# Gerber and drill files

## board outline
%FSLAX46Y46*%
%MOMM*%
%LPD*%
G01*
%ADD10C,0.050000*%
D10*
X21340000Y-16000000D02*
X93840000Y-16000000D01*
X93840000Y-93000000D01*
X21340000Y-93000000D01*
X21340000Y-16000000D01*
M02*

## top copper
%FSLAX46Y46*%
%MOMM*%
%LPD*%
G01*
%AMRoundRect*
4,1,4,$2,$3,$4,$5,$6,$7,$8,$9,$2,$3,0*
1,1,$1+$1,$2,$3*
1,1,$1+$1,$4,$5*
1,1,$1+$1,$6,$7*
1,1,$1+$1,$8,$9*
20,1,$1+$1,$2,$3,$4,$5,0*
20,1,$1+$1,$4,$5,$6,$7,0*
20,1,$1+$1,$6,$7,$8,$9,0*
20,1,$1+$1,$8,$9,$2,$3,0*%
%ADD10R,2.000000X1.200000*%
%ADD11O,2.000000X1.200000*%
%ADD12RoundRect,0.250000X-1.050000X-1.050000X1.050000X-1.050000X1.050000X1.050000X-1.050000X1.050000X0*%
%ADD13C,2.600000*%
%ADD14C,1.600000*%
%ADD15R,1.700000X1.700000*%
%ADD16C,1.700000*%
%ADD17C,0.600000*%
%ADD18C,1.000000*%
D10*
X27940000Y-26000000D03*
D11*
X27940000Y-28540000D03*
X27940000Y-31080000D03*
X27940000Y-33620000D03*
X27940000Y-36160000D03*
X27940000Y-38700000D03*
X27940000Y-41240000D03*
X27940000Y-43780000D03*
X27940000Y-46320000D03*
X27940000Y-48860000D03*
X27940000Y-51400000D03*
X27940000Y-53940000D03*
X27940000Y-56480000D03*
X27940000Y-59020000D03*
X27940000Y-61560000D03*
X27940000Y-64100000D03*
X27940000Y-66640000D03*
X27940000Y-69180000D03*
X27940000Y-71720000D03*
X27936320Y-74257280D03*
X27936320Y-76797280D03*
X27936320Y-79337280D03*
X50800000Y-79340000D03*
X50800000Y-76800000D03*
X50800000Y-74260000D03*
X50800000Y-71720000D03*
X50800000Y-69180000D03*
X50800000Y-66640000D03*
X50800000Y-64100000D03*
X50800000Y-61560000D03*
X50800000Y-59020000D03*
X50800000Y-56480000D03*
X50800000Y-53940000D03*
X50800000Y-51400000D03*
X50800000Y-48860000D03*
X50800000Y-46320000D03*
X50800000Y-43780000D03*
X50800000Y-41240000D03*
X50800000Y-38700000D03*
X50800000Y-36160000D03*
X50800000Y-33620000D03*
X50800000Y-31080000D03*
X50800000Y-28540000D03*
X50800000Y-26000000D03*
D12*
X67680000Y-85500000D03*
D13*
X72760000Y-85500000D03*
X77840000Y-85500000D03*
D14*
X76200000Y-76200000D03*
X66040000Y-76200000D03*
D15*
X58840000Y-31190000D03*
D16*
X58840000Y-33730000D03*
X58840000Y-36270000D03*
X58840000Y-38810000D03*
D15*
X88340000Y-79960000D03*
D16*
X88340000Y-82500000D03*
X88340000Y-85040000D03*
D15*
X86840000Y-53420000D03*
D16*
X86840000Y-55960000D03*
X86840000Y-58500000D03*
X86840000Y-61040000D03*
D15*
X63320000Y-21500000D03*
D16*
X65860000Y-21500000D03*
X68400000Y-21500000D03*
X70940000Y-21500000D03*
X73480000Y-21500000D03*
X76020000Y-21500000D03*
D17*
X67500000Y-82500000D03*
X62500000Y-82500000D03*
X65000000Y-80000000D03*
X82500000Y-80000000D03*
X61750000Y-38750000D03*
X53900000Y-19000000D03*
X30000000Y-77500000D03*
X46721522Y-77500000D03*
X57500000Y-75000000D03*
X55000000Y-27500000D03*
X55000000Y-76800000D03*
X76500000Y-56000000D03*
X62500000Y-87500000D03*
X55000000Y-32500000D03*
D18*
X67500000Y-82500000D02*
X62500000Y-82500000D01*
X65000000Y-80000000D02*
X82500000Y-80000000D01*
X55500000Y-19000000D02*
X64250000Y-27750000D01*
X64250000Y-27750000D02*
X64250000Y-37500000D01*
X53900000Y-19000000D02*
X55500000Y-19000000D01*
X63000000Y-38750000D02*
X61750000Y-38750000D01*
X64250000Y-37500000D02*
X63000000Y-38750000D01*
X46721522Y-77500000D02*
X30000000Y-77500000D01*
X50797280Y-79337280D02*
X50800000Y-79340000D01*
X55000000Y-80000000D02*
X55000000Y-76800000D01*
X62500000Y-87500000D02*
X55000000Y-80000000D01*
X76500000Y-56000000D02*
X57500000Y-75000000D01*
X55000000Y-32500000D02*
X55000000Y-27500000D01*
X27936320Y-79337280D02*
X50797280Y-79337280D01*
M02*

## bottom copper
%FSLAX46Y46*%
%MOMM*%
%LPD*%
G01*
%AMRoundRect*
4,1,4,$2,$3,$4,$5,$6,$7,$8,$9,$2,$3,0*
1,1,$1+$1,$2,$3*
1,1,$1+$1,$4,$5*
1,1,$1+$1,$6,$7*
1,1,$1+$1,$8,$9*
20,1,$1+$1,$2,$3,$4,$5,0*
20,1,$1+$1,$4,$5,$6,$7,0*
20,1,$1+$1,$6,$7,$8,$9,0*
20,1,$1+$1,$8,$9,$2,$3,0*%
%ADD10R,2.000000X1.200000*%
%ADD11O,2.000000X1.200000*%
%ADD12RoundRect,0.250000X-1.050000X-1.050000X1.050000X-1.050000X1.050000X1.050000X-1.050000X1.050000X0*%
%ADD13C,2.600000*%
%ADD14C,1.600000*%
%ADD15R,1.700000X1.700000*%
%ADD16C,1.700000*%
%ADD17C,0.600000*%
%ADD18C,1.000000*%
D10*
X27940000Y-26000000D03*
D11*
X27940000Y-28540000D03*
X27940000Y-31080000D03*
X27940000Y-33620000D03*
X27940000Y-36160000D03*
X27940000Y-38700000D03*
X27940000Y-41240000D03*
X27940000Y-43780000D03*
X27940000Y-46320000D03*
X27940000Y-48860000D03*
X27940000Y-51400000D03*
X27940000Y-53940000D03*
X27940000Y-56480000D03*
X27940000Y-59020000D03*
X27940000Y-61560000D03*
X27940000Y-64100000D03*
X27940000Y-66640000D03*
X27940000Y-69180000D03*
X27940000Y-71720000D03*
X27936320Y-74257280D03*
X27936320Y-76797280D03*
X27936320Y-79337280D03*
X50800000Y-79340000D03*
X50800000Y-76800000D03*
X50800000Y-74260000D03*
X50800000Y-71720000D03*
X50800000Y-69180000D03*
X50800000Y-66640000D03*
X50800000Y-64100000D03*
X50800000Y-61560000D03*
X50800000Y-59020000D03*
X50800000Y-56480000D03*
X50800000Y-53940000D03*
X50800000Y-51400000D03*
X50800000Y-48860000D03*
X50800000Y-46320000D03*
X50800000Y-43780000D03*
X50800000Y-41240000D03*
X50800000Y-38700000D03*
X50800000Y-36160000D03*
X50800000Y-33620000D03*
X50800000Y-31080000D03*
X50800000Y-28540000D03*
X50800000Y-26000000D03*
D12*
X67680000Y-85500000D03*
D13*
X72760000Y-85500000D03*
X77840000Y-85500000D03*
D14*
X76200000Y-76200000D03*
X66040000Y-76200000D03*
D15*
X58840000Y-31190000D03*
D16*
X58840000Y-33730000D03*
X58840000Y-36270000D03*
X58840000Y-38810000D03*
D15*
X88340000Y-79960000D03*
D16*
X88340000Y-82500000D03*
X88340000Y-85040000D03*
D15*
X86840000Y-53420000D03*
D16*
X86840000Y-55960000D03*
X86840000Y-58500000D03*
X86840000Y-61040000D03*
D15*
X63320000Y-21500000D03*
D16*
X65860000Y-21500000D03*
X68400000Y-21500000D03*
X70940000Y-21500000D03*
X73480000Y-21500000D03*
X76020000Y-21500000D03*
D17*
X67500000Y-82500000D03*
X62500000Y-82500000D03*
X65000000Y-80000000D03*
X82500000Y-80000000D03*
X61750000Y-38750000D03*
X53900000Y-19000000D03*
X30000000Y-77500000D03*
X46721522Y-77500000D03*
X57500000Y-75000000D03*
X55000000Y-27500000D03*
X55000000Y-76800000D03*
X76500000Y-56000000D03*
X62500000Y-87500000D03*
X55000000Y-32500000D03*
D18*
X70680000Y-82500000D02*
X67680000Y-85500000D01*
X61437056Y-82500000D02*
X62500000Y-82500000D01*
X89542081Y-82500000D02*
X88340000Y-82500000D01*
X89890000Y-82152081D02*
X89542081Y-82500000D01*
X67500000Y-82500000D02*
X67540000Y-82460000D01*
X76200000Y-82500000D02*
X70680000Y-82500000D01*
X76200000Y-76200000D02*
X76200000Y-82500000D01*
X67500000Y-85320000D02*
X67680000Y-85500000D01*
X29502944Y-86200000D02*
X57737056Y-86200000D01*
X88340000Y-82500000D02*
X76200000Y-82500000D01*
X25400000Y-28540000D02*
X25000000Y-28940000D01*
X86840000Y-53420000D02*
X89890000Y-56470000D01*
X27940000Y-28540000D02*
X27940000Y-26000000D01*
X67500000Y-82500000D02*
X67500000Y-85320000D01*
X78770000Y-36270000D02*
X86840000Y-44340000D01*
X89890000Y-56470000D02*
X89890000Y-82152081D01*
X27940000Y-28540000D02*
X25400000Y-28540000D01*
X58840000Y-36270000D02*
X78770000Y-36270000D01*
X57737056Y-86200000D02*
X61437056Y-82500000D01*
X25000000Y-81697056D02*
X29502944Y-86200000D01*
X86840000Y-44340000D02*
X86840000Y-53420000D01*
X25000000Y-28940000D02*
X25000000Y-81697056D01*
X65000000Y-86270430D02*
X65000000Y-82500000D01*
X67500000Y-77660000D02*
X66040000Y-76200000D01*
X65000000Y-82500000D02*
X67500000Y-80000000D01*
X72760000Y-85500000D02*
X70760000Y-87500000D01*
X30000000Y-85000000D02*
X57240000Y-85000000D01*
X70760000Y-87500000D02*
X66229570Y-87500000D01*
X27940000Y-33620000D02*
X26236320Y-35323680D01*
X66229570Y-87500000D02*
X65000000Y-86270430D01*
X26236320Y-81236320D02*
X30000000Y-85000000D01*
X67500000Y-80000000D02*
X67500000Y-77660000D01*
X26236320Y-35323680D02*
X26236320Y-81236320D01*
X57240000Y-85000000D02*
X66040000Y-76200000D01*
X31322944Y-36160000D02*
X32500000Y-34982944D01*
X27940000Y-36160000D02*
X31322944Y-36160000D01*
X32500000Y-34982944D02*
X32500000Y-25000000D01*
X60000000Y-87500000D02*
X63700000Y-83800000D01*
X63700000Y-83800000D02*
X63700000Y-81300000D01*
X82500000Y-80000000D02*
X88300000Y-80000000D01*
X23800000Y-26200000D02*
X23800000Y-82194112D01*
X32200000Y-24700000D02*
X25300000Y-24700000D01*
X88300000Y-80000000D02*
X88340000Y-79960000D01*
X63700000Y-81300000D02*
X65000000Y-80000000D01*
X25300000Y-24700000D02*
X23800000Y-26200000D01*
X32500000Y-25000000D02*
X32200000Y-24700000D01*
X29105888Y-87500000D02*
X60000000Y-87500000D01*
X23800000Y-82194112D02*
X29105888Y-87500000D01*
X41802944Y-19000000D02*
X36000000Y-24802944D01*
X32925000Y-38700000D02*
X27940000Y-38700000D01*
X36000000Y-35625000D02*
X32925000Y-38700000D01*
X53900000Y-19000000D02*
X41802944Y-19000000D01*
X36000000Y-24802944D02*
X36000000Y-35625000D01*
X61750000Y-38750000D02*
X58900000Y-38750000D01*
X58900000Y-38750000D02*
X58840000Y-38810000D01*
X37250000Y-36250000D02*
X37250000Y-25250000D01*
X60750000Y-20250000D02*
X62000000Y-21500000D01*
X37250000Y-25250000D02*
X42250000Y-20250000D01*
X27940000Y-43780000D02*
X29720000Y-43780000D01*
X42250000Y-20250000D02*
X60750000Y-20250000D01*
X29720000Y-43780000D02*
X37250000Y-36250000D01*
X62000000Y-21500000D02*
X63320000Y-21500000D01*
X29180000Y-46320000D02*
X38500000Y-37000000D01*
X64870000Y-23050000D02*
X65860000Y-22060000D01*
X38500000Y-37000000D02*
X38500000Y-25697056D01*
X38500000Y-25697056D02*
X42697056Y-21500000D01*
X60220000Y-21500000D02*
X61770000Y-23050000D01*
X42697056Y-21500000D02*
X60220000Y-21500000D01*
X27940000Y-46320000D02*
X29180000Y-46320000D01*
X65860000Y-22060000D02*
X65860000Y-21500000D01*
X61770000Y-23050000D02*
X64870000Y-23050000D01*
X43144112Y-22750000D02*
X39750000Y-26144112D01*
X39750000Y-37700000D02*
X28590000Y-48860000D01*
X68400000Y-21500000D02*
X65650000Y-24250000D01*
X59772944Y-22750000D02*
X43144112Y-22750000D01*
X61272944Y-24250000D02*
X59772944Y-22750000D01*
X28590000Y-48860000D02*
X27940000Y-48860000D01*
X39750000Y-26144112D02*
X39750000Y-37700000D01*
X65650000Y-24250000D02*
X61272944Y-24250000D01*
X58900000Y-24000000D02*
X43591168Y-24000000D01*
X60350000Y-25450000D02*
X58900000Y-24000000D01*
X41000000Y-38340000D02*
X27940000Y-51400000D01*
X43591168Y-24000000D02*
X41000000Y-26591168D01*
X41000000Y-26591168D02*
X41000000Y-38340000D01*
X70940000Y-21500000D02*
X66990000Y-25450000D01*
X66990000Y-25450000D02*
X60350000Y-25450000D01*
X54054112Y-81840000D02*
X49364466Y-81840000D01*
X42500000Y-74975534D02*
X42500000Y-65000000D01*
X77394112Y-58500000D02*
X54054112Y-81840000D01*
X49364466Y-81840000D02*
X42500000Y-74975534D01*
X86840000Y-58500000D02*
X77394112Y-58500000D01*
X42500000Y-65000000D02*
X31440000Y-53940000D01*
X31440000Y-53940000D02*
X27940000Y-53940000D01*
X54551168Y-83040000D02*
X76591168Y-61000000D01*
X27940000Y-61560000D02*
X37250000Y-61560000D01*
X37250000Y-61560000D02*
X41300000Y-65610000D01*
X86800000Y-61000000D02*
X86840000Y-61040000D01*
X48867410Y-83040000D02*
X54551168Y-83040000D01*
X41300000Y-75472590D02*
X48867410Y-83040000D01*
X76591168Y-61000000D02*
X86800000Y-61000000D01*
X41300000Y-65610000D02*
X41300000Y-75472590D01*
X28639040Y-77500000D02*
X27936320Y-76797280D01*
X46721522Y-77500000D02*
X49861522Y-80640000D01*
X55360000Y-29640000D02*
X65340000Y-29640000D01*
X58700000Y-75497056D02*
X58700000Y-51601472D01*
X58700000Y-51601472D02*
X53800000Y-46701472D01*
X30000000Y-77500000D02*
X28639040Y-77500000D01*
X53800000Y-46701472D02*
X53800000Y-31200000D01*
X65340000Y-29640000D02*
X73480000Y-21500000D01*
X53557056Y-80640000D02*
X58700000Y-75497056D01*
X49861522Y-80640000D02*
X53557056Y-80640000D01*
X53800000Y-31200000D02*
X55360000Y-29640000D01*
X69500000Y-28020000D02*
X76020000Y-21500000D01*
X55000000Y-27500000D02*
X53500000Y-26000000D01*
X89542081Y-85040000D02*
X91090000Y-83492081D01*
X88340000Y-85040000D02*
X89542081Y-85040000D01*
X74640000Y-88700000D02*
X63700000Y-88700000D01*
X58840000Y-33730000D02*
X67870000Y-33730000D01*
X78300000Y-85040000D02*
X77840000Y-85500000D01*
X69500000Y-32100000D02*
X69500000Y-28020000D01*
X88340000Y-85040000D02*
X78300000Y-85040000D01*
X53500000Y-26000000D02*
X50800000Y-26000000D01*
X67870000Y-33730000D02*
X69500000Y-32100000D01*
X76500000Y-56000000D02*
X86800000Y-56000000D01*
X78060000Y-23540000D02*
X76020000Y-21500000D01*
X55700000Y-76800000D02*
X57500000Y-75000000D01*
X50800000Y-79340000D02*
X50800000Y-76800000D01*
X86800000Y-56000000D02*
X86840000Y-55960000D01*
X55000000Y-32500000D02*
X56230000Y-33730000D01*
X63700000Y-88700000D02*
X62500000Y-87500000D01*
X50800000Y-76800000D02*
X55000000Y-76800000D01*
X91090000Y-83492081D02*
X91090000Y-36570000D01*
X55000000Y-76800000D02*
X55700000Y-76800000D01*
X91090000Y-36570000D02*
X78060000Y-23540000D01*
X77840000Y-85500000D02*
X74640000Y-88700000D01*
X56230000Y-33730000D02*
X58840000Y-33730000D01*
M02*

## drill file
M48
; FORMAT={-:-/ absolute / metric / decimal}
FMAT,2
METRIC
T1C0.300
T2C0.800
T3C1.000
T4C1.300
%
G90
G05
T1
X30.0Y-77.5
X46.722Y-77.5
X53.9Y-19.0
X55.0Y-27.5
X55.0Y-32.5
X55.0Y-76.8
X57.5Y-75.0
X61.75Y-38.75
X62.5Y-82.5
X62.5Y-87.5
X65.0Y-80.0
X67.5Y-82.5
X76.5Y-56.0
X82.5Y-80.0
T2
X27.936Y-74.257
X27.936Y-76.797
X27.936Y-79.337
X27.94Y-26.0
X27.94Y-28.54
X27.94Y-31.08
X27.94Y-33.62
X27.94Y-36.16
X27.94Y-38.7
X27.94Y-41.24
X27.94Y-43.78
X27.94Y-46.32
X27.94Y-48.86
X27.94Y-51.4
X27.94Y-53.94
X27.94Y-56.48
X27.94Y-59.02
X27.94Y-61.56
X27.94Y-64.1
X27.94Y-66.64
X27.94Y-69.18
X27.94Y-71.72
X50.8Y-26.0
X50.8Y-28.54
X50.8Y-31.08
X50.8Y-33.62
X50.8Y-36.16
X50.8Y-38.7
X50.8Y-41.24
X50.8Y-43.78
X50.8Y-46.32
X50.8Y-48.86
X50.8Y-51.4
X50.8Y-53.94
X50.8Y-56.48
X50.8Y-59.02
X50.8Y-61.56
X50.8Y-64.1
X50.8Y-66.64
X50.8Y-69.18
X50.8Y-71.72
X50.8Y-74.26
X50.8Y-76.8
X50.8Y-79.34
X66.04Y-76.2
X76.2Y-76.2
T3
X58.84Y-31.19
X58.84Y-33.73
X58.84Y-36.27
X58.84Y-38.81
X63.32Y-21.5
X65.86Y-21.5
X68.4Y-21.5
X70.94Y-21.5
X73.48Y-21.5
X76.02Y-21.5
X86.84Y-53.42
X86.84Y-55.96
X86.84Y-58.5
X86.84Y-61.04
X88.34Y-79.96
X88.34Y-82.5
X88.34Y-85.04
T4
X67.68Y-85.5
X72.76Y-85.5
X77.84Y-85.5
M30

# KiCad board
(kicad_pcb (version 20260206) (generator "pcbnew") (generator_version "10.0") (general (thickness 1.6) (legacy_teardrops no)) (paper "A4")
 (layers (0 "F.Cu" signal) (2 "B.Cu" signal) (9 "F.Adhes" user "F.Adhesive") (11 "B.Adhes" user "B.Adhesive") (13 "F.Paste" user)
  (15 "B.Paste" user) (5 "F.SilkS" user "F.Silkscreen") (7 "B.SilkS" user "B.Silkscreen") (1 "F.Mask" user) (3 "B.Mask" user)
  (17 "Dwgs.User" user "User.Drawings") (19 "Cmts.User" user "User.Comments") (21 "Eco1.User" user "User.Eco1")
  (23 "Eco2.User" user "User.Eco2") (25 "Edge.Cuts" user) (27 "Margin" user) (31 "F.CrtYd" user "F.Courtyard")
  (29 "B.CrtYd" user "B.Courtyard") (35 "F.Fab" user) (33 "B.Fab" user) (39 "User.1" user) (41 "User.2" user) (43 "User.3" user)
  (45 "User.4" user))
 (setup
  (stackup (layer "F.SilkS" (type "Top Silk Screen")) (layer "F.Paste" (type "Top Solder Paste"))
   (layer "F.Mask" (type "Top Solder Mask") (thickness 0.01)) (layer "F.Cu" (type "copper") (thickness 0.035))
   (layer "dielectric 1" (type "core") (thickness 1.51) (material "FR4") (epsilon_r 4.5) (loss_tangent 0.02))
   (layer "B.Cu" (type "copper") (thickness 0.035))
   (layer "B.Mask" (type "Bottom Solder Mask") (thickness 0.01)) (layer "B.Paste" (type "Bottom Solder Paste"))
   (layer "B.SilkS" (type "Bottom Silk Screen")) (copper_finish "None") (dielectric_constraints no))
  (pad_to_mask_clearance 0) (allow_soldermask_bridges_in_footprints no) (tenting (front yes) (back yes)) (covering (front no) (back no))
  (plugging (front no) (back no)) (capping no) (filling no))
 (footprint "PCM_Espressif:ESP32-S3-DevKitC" (layer "F.Cu") (at 27.94 26)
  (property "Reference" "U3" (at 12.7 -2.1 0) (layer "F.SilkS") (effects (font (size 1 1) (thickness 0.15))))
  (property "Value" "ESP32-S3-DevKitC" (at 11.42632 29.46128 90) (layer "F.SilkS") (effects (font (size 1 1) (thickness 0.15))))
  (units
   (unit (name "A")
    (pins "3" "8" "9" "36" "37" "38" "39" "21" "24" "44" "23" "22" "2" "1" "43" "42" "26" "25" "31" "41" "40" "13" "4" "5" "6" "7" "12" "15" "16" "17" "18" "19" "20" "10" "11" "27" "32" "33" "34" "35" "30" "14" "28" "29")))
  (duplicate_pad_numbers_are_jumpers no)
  (pad "1" thru_hole rect (at 0 0 270) (size 1.2 2) (drill 0.8) (layers "*.Cu" "*.Mask") (remove_unused_layers no) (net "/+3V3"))
  (pad "2" thru_hole oval (at 0 2.54 270) (size 1.2 2) (drill 0.8) (layers "*.Cu" "*.Mask") (remove_unused_layers no) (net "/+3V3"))
  (pad "3" thru_hole oval (at 0 5.08 270) (size 1.2 2) (drill 0.8) (layers "*.Cu" "*.Mask") (remove_unused_layers no)
   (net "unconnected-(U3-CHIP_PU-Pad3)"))
  (pad "4" thru_hole oval (at 0 7.62 270) (size 1.2 2) (drill 0.8) (layers "*.Cu" "*.Mask") (remove_unused_layers no) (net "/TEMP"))
  (pad "5" thru_hole oval (at 0 10.16 270) (size 1.2 2) (drill 0.8) (layers "*.Cu" "*.Mask") (remove_unused_layers no) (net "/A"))
  (pad "6" thru_hole oval (at 0 12.7 270) (size 1.2 2) (drill 0.8) (layers "*.Cu" "*.Mask") (remove_unused_layers no) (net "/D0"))
  (pad "7" thru_hole oval (at 0 15.24 270) (size 1.2 2) (drill 0.8) (layers "*.Cu" "*.Mask") (remove_unused_layers no)
   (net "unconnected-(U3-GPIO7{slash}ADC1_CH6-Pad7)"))
  (pad "8" thru_hole oval (at 0 17.78 270) (size 1.2 2) (drill 0.8) (layers "*.Cu" "*.Mask") (remove_unused_layers no) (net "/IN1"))
  (pad "9" thru_hole oval (at 0 20.32 270) (size 1.2 2) (drill 0.8) (layers "*.Cu" "*.Mask") (remove_unused_layers no) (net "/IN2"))
  (pad "10" thru_hole oval (at 0 22.86 270) (size 1.2 2) (drill 0.8) (layers "*.Cu" "*.Mask") (remove_unused_layers no) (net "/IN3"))
  (pad "11" thru_hole oval (at 0 25.4 270) (size 1.2 2) (drill 0.8) (layers "*.Cu" "*.Mask") (remove_unused_layers no) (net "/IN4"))
  (pad "12" thru_hole oval (at 0 27.94 270) (size 1.2 2) (drill 0.8) (layers "*.Cu" "*.Mask") (remove_unused_layers no) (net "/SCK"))
  (pad "13" thru_hole oval (at 0 30.48 270) (size 1.2 2) (drill 0.8) (layers "*.Cu" "*.Mask") (remove_unused_layers no)
   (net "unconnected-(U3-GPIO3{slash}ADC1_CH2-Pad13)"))
  (pad "14" thru_hole oval (at 0 33.02 270) (size 1.2 2) (drill 0.8) (layers "*.Cu" "*.Mask") (remove_unused_layers no)
   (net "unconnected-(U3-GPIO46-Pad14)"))
  (pad "15" thru_hole oval (at 0 35.56 270) (size 1.2 2) (drill 0.8) (layers "*.Cu" "*.Mask") (remove_unused_layers no) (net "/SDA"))
  (pad "16" thru_hole oval (at 0 38.1 270) (size 1.2 2) (drill 0.8) (layers "*.Cu" "*.Mask") (remove_unused_layers no)
   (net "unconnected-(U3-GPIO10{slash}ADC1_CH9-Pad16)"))
  (pad "17" thru_hole oval (at 0 40.64 270) (size 1.2 2) (drill 0.8) (layers "*.Cu" "*.Mask") (remove_unused_layers no)
   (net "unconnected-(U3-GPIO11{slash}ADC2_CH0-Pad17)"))
  (pad "18" thru_hole oval (at 0 43.18 270) (size 1.2 2) (drill 0.8) (layers "*.Cu" "*.Mask") (remove_unused_layers no)
   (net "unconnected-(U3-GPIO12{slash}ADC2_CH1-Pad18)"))
  (pad "19" thru_hole oval (at 0 45.72 270) (size 1.2 2) (drill 0.8) (layers "*.Cu" "*.Mask") (remove_unused_layers no)
   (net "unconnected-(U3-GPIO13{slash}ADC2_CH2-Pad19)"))
  (pad "20" thru_hole oval (at -0.00368 48.25728 270) (size 1.2 2) (drill 0.8) (layers "*.Cu" "*.Mask") (remove_unused_layers no)
   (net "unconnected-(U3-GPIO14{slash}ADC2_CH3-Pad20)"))
  (pad "21" thru_hole oval (at -0.00368 50.79728 270) (size 1.2 2) (drill 0.8) (layers "*.Cu" "*.Mask") (remove_unused_layers no)
   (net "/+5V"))
  (pad "22" thru_hole oval (at -0.00368 53.33728 270) (size 1.2 2) (drill 0.8) (layers "*.Cu" "*.Mask") (remove_unused_layers no)
   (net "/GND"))
  (pad "23" thru_hole oval (at 22.86 53.34 270) (size 1.2 2) (drill 0.8) (layers "*.Cu" "*.Mask") (remove_unused_layers no) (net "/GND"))
  (pad "24" thru_hole oval (at 22.86 50.8 270) (size 1.2 2) (drill 0.8) (layers "*.Cu" "*.Mask") (remove_unused_layers no) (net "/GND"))
  (pad "25" thru_hole oval (at 22.86 48.26 270) (size 1.2 2) (drill 0.8) (layers "*.Cu" "*.Mask") (remove_unused_layers no)
   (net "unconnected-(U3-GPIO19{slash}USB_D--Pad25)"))
  (pad "26" thru_hole oval (at 22.86 45.72 270) (size 1.2 2) (drill 0.8) (layers "*.Cu" "*.Mask") (remove_unused_layers no)
   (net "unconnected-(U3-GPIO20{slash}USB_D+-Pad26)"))
  (pad "27" thru_hole oval (at 22.86 43.18 270) (size 1.2 2) (drill 0.8) (layers "*.Cu" "*.Mask") (remove_unused_layers no)
   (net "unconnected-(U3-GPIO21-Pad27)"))
  (pad "28" thru_hole oval (at 22.86 40.64 270) (size 1.2 2) (drill 0.8) (layers "*.Cu" "*.Mask") (remove_unused_layers no)
   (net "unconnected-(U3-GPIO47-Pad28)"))
  (pad "29" thru_hole oval (at 22.86 38.1 270) (size 1.2 2) (drill 0.8) (layers "*.Cu" "*.Mask") (remove_unused_layers no)
   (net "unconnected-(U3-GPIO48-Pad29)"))
  (pad "30" thru_hole oval (at 22.86 35.56 270) (size 1.2 2) (drill 0.8) (layers "*.Cu" "*.Mask") (remove_unused_layers no)
   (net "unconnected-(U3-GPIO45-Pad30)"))
  (pad "31" thru_hole oval (at 22.86 33.02 270) (size 1.2 2) (drill 0.8) (layers "*.Cu" "*.Mask") (remove_unused_layers no)
   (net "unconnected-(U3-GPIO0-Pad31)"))
  (pad "32" thru_hole oval (at 22.86 30.48 270) (size 1.2 2) (drill 0.8) (layers "*.Cu" "*.Mask") (remove_unused_layers no)
   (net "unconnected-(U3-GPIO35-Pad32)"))
  (pad "33" thru_hole oval (at 22.86 27.94 270) (size 1.2 2) (drill 0.8) (layers "*.Cu" "*.Mask") (remove_unused_layers no)
   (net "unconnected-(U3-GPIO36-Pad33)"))
  (pad "34" thru_hole oval (at 22.86 25.4 270) (size 1.2 2) (drill 0.8) (layers "*.Cu" "*.Mask") (remove_unused_layers no)
   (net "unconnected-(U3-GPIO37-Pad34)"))
  (pad "35" thru_hole oval (at 22.86 22.86 270) (size 1.2 2) (drill 0.8) (layers "*.Cu" "*.Mask") (remove_unused_layers no)
   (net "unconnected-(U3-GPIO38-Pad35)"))
  (pad "36" thru_hole oval (at 22.86 20.32 270) (size 1.2 2) (drill 0.8) (layers "*.Cu" "*.Mask") (remove_unused_layers no)
   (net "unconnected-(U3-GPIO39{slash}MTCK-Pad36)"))
  (pad "37" thru_hole oval (at 22.86 17.78 270) (size 1.2 2) (drill 0.8) (layers "*.Cu" "*.Mask") (remove_unused_layers no)
   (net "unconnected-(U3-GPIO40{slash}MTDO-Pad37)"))
  (pad "38" thru_hole oval (at 22.86 15.24 270) (size 1.2 2) (drill 0.8) (layers "*.Cu" "*.Mask") (remove_unused_layers no)
   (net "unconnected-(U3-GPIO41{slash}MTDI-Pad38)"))
  (pad "39" thru_hole oval (at 22.86 12.7 270) (size 1.2 2) (drill 0.8) (layers "*.Cu" "*.Mask") (remove_unused_layers no)
   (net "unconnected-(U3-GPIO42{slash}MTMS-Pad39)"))
  (pad "40" thru_hole oval (at 22.86 10.16 270) (size 1.2 2) (drill 0.8) (layers "*.Cu" "*.Mask") (remove_unused_layers no)
   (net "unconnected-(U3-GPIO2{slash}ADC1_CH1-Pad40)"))
  (pad "41" thru_hole oval (at 22.86 7.62 270) (size 1.2 2) (drill 0.8) (layers "*.Cu" "*.Mask") (remove_unused_layers no)
   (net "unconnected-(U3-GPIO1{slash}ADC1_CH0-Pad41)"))
  (pad "42" thru_hole oval (at 22.86 5.08 270) (size 1.2 2) (drill 0.8) (layers "*.Cu" "*.Mask") (remove_unused_layers no)
   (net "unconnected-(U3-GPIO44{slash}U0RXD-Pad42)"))
  (pad "43" thru_hole oval (at 22.86 2.54 270) (size 1.2 2) (drill 0.8) (layers "*.Cu" "*.Mask") (remove_unused_layers no)
   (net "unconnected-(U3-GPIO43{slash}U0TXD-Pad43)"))
  (pad "44" thru_hole oval (at 22.86 0 270) (size 1.2 2) (drill 0.8) (layers "*.Cu" "*.Mask") (remove_unused_layers no) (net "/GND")))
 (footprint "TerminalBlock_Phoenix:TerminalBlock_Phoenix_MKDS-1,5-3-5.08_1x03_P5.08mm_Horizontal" (layer "F.Cu") (at 67.68 85.5)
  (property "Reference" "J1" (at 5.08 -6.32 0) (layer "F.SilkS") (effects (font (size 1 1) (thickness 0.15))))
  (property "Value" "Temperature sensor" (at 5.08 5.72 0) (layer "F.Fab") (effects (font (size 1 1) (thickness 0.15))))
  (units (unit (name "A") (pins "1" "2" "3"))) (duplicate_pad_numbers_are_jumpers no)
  (pad "1" thru_hole roundrect (at 0 0) (size 2.6 2.6) (drill 1.3) (layers "*.Cu" "*.Mask") (remove_unused_layers no)
   (roundrect_rratio 0.096154) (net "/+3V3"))
  (pad "2" thru_hole circle (at 5.08 0) (size 2.6 2.6) (drill 1.3) (layers "*.Cu" "*.Mask") (remove_unused_layers no) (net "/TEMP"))
  (pad "3" thru_hole circle (at 10.16 0) (size 2.6 2.6) (drill 1.3) (layers "*.Cu" "*.Mask") (remove_unused_layers no) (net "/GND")))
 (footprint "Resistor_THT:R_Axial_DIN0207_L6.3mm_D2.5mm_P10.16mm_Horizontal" (layer "F.Cu") (at 76.2 76.2 180)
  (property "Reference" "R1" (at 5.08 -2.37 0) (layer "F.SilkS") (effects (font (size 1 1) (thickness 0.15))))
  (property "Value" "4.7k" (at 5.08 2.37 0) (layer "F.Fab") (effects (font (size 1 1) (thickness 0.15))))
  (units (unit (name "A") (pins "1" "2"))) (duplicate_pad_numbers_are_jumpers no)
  (pad "1" thru_hole circle (at 0 0 180) (size 1.6 1.6) (drill 0.8) (layers "*.Cu" "*.Mask") (remove_unused_layers no) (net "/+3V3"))
  (pad "2" thru_hole circle (at 10.16 0 180) (size 1.6 1.6) (drill 0.8) (layers "*.Cu" "*.Mask") (remove_unused_layers no) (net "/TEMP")))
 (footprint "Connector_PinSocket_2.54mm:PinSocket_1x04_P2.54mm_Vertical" (layer "F.Cu") (at 58.84 31.19)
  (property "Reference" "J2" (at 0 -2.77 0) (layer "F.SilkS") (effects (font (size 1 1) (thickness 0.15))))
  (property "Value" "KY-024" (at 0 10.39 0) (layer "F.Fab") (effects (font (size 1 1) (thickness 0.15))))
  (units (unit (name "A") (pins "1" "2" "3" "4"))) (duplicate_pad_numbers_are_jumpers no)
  (pad "1" thru_hole rect (at 0 0) (size 1.7 1.7) (drill 1) (layers "*.Cu" "*.Mask") (remove_unused_layers no)
   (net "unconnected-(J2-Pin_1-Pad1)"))
  (pad "2" thru_hole circle (at 0 2.54) (size 1.7 1.7) (drill 1) (layers "*.Cu" "*.Mask") (remove_unused_layers no) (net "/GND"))
  (pad "3" thru_hole circle (at 0 5.08) (size 1.7 1.7) (drill 1) (layers "*.Cu" "*.Mask") (remove_unused_layers no) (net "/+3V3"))
  (pad "4" thru_hole circle (at 0 7.62) (size 1.7 1.7) (drill 1) (layers "*.Cu" "*.Mask") (remove_unused_layers no) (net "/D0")))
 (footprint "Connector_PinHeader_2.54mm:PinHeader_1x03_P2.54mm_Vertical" (layer "F.Cu") (at 88.34 79.96)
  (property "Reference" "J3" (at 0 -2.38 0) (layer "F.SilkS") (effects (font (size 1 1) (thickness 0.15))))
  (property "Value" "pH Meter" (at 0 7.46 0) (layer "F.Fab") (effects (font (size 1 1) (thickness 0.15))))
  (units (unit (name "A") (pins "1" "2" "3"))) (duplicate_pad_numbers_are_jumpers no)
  (pad "1" thru_hole rect (at 0 0) (size 1.7 1.7) (drill 1) (layers "*.Cu" "*.Mask") (remove_unused_layers no) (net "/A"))
  (pad "2" thru_hole circle (at 0 2.54) (size 1.7 1.7) (drill 1) (layers "*.Cu" "*.Mask") (remove_unused_layers no) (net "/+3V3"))
  (pad "3" thru_hole circle (at 0 5.08) (size 1.7 1.7) (drill 1) (layers "*.Cu" "*.Mask") (remove_unused_layers no) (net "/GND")))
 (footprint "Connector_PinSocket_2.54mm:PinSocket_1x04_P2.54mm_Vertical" (layer "F.Cu") (at 86.84 53.42)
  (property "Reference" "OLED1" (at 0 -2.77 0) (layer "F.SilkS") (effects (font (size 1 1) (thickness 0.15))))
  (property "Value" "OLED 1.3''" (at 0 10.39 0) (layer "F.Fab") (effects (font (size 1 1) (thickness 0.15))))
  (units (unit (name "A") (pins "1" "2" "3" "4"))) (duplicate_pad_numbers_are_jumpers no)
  (pad "1" thru_hole rect (at 0 0) (size 1.7 1.7) (drill 1) (layers "*.Cu" "*.Mask") (remove_unused_layers no) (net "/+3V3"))
  (pad "2" thru_hole circle (at 0 2.54) (size 1.7 1.7) (drill 1) (layers "*.Cu" "*.Mask") (remove_unused_layers no) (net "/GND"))
  (pad "3" thru_hole circle (at 0 5.08) (size 1.7 1.7) (drill 1) (layers "*.Cu" "*.Mask") (remove_unused_layers no) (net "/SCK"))
  (pad "4" thru_hole circle (at 0 7.62) (size 1.7 1.7) (drill 1) (layers "*.Cu" "*.Mask") (remove_unused_layers no) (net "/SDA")))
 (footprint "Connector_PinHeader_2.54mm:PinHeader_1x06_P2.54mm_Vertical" (layer "F.Cu") (at 63.32 21.5 90)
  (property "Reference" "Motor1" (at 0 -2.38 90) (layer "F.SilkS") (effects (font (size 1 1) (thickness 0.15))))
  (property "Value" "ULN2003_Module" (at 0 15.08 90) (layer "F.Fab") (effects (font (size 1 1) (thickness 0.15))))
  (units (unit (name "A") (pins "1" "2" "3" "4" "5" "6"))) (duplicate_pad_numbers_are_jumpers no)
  (pad "1" thru_hole rect (at 0 0 90) (size 1.7 1.7) (drill 1) (layers "*.Cu" "*.Mask") (remove_unused_layers no) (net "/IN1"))
  (pad "2" thru_hole circle (at 0 2.54 90) (size 1.7 1.7) (drill 1) (layers "*.Cu" "*.Mask") (remove_unused_layers no) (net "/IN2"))
  (pad "3" thru_hole circle (at 0 5.08 90) (size 1.7 1.7) (drill 1) (layers "*.Cu" "*.Mask") (remove_unused_layers no) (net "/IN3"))
  (pad "4" thru_hole circle (at 0 7.62 90) (size 1.7 1.7) (drill 1) (layers "*.Cu" "*.Mask") (remove_unused_layers no) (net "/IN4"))
  (pad "5" thru_hole circle (at 0 10.16 90) (size 1.7 1.7) (drill 1) (layers "*.Cu" "*.Mask") (remove_unused_layers no) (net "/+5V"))
  (pad "6" thru_hole circle (at 0 12.7 90) (size 1.7 1.7) (drill 1) (layers "*.Cu" "*.Mask") (remove_unused_layers no) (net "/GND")))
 (gr_rect (start 21.34 16) (end 93.84 93) (stroke (width 0.05) (type default)) (fill no) (layer "Edge.Cuts"))
 (segment (start 67.5 82.5) (end 62.5 82.5) (width 1) (layer "F.Cu") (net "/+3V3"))
 (via (at 67.5 82.5) (size 0.6) (drill 0.3) (layers "F.Cu" "B.Cu") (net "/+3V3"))
 (via (at 62.5 82.5) (size 0.6) (drill 0.3) (layers "F.Cu" "B.Cu") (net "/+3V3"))
 (segment (start 70.68 82.5) (end 67.68 85.5) (width 1) (layer "B.Cu") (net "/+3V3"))
 (segment (start 61.437056 82.5) (end 62.5 82.5) (width 1) (layer "B.Cu") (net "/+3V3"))
 (segment (start 89.542081 82.5) (end 88.34 82.5) (width 1) (layer "B.Cu") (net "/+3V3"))
 (segment (start 89.89 82.152081) (end 89.542081 82.5) (width 1) (layer "B.Cu") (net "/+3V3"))
 (segment (start 67.5 82.5) (end 67.54 82.46) (width 1) (layer "B.Cu") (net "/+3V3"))
 (segment (start 76.2 82.5) (end 70.68 82.5) (width 1) (layer "B.Cu") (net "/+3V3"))
 (segment (start 76.2 76.2) (end 76.2 82.5) (width 1) (layer "B.Cu") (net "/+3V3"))
 (segment (start 67.5 85.32) (end 67.68 85.5) (width 1) (layer "B.Cu") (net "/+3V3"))
 (segment (start 29.502944 86.2) (end 57.737056 86.2) (width 1) (layer "B.Cu") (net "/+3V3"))
 (segment (start 88.34 82.5) (end 76.2 82.5) (width 1) (layer "B.Cu") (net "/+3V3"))
 (segment (start 25.4 28.54) (end 25 28.94) (width 1) (layer "B.Cu") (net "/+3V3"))
 (segment (start 86.84 53.42) (end 89.89 56.47) (width 1) (layer "B.Cu") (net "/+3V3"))
 (segment (start 27.94 28.54) (end 27.94 26) (width 1) (layer "B.Cu") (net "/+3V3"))
 (segment (start 67.5 82.5) (end 67.5 85.32) (width 1) (layer "B.Cu") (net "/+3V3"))
 (segment (start 78.77 36.27) (end 86.84 44.34) (width 1) (layer "B.Cu") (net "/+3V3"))
 (segment (start 89.89 56.47) (end 89.89 82.152081) (width 1) (layer "B.Cu") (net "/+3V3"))
 (segment (start 27.94 28.54) (end 25.4 28.54) (width 1) (layer "B.Cu") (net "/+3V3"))
 (segment (start 58.84 36.27) (end 78.77 36.27) (width 1) (layer "B.Cu") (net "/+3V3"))
 (segment (start 57.737056 86.2) (end 61.437056 82.5) (width 1) (layer "B.Cu") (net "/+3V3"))
 (segment (start 25 81.697056) (end 29.502944 86.2) (width 1) (layer "B.Cu") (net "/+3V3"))
 (segment (start 86.84 44.34) (end 86.84 53.42) (width 1) (layer "B.Cu") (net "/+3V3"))
 (segment (start 25 28.94) (end 25 81.697056) (width 1) (layer "B.Cu") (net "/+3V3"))
 (segment (start 65 86.27043) (end 65 82.5) (width 1) (layer "B.Cu") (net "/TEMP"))
 (segment (start 67.5 77.66) (end 66.04 76.2) (width 1) (layer "B.Cu") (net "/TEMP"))
 (segment (start 65 82.5) (end 67.5 80) (width 1) (layer "B.Cu") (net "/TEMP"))
 (segment (start 72.76 85.5) (end 70.76 87.5) (width 1) (layer "B.Cu") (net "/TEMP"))
 (segment (start 30 85) (end 57.24 85) (width 1) (layer "B.Cu") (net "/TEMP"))
 (segment (start 70.76 87.5) (end 66.22957 87.5) (width 1) (layer "B.Cu") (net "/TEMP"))
 (segment (start 27.94 33.62) (end 26.23632 35.32368) (width 1) (layer "B.Cu") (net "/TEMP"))
 (segment (start 66.22957 87.5) (end 65 86.27043) (width 1) (layer "B.Cu") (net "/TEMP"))
 (segment (start 26.23632 81.23632) (end 30 85) (width 1) (layer "B.Cu") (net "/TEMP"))
 (segment (start 67.5 80) (end 67.5 77.66) (width 1) (layer "B.Cu") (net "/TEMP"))
 (segment (start 26.23632 35.32368) (end 26.23632 81.23632) (width 1) (layer "B.Cu") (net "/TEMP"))
 (segment (start 57.24 85) (end 66.04 76.2) (width 1) (layer "B.Cu") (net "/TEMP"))
 (segment (start 65 80) (end 82.5 80) (width 1) (layer "F.Cu") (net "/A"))
 (via (at 65 80) (size 0.6) (drill 0.3) (layers "F.Cu" "B.Cu") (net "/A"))
 (via (at 82.5 80) (size 0.6) (drill 0.3) (layers "F.Cu" "B.Cu") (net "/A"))
 (segment (start 31.322944 36.16) (end 32.5 34.982944) (width 1) (layer "B.Cu") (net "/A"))
 (segment (start 27.94 36.16) (end 31.322944 36.16) (width 1) (layer "B.Cu") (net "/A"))
 (segment (start 32.5 34.982944) (end 32.5 25) (width 1) (layer "B.Cu") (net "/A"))
 (segment (start 60 87.5) (end 63.7 83.8) (width 1) (layer "B.Cu") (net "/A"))
 (segment (start 63.7 83.8) (end 63.7 81.3) (width 1) (layer "B.Cu") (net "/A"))
 (segment (start 82.5 80) (end 88.3 80) (width 1) (layer "B.Cu") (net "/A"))
 (segment (start 23.8 26.2) (end 23.8 82.194112) (width 1) (layer "B.Cu") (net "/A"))
 (segment (start 32.2 24.7) (end 25.3 24.7) (width 1) (layer "B.Cu") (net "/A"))
 (segment (start 88.3 80) (end 88.34 79.96) (width 1) (layer "B.Cu") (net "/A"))
 (segment (start 63.7 81.3) (end 65 80) (width 1) (layer "B.Cu") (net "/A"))
 (segment (start 25.3 24.7) (end 23.8 26.2) (width 1) (layer "B.Cu") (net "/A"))
 (segment (start 32.5 25) (end 32.2 24.7) (width 1) (layer "B.Cu") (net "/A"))
 (segment (start 29.105888 87.5) (end 60 87.5) (width 1) (layer "B.Cu") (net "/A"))
 (segment (start 23.8 82.194112) (end 29.105888 87.5) (width 1) (layer "B.Cu") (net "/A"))
 (segment (start 55.5 19) (end 64.25 27.75) (width 1) (layer "F.Cu") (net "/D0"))
 (segment (start 64.25 27.75) (end 64.25 37.5) (width 1) (layer "F.Cu") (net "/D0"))
 (segment (start 53.9 19) (end 55.5 19) (width 1) (layer "F.Cu") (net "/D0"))
 (segment (start 63 38.75) (end 61.75 38.75) (width 1) (layer "F.Cu") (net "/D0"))
 (segment (start 64.25 37.5) (end 63 38.75) (width 1) (layer "F.Cu") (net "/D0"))
 (via (at 61.75 38.75) (size 0.6) (drill 0.3) (layers "F.Cu" "B.Cu") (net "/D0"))
 (via (at 53.9 19) (size 0.6) (drill 0.3) (layers "F.Cu" "B.Cu") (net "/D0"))
 (segment (start 41.802944 19) (end 36 24.802944) (width 1) (layer "B.Cu") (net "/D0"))
 (segment (start 32.925 38.7) (end 27.94 38.7) (width 1) (layer "B.Cu") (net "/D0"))
 (segment (start 36 35.625) (end 32.925 38.7) (width 1) (layer "B.Cu") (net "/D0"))
 (segment (start 53.9 19) (end 41.802944 19) (width 1) (layer "B.Cu") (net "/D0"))
 (segment (start 36 24.802944) (end 36 35.625) (width 1) (layer "B.Cu") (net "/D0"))
 (segment (start 61.75 38.75) (end 58.9 38.75) (width 1) (layer "B.Cu") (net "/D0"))
 (segment (start 58.9 38.75) (end 58.84 38.81) (width 1) (layer "B.Cu") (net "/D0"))
 (segment (start 37.25 36.25) (end 37.25 25.25) (width 1) (layer "B.Cu") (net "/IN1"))
 (segment (start 60.75 20.25) (end 62 21.5) (width 1) (layer "B.Cu") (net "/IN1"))
 (segment (start 37.25 25.25) (end 42.25 20.25) (width 1) (layer "B.Cu") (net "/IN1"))
 (segment (start 27.94 43.78) (end 29.72 43.78) (width 1) (layer "B.Cu") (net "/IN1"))
 (segment (start 42.25 20.25) (end 60.75 20.25) (width 1) (layer "B.Cu") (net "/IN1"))
 (segment (start 29.72 43.78) (end 37.25 36.25) (width 1) (layer "B.Cu") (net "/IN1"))
 (segment (start 62 21.5) (end 63.32 21.5) (width 1) (layer "B.Cu") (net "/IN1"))
 (segment (start 29.18 46.32) (end 38.5 37) (width 1) (layer "B.Cu") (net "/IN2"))
 (segment (start 64.87 23.05) (end 65.86 22.06) (width 1) (layer "B.Cu") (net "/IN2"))
 (segment (start 38.5 37) (end 38.5 25.697056) (width 1) (layer "B.Cu") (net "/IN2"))
 (segment (start 38.5 25.697056) (end 42.697056 21.5) (width 1) (layer "B.Cu") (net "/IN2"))
 (segment (start 60.22 21.5) (end 61.77 23.05) (width 1) (layer "B.Cu") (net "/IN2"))
 (segment (start 42.697056 21.5) (end 60.22 21.5) (width 1) (layer "B.Cu") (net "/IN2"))
 (segment (start 27.94 46.32) (end 29.18 46.32) (width 1) (layer "B.Cu") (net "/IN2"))
 (segment (start 65.86 22.06) (end 65.86 21.5) (width 1) (layer "B.Cu") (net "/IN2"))
 (segment (start 61.77 23.05) (end 64.87 23.05) (width 1) (layer "B.Cu") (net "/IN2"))
 (segment (start 43.144112 22.75) (end 39.75 26.144112) (width 1) (layer "B.Cu") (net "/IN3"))
 (segment (start 39.75 37.7) (end 28.59 48.86) (width 1) (layer "B.Cu") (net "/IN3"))
 (segment (start 68.4 21.5) (end 65.65 24.25) (width 1) (layer "B.Cu") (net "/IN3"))
 (segment (start 59.772944 22.75) (end 43.144112 22.75) (width 1) (layer "B.Cu") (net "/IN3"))
 (segment (start 61.272944 24.25) (end 59.772944 22.75) (width 1) (layer "B.Cu") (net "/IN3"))
 (segment (start 28.59 48.86) (end 27.94 48.86) (width 1) (layer "B.Cu") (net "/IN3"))
 (segment (start 39.75 26.144112) (end 39.75 37.7) (width 1) (layer "B.Cu") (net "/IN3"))
 (segment (start 65.65 24.25) (end 61.272944 24.25) (width 1) (layer "B.Cu") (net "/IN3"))
 (segment (start 58.9 24) (end 43.591168 24) (width 1) (layer "B.Cu") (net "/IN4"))
 (segment (start 60.35 25.45) (end 58.9 24) (width 1) (layer "B.Cu") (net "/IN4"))
 (segment (start 41 38.34) (end 27.94 51.4) (width 1) (layer "B.Cu") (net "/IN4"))
 (segment (start 43.591168 24) (end 41 26.591168) (width 1) (layer "B.Cu") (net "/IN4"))
 (segment (start 41 26.591168) (end 41 38.34) (width 1) (layer "B.Cu") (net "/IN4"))
 (segment (start 70.94 21.5) (end 66.99 25.45) (width 1) (layer "B.Cu") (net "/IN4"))
 (segment (start 66.99 25.45) (end 60.35 25.45) (width 1) (layer "B.Cu") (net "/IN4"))
 (segment (start 54.054112 81.84) (end 49.364466 81.84) (width 1) (layer "B.Cu") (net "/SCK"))
 (segment (start 42.5 74.975534) (end 42.5 65) (width 1) (layer "B.Cu") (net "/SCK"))
 (segment (start 77.394112 58.5) (end 54.054112 81.84) (width 1) (layer "B.Cu") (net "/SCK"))
 (segment (start 49.364466 81.84) (end 42.5 74.975534) (width 1) (layer "B.Cu") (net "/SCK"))
 (segment (start 86.84 58.5) (end 77.394112 58.5) (width 1) (layer "B.Cu") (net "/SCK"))
 (segment (start 42.5 65) (end 31.44 53.94) (width 1) (layer "B.Cu") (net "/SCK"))
 (segment (start 31.44 53.94) (end 27.94 53.94) (width 1) (layer "B.Cu") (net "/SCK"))
 (segment (start 54.551168 83.04) (end 76.591168 61) (width 1) (layer "B.Cu") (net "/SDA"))
 (segment (start 27.94 61.56) (end 37.25 61.56) (width 1) (layer "B.Cu") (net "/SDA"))
 (segment (start 37.25 61.56) (end 41.3 65.61) (width 1) (layer "B.Cu") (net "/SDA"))
 (segment (start 86.8 61) (end 86.84 61.04) (width 1) (layer "B.Cu") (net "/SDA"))
 (segment (start 48.86741 83.04) (end 54.551168 83.04) (width 1) (layer "B.Cu") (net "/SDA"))
 (segment (start 41.3 75.47259) (end 48.86741 83.04) (width 1) (layer "B.Cu") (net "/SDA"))
 (segment (start 76.591168 61) (end 86.8 61) (width 1) (layer "B.Cu") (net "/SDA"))
 (segment (start 41.3 65.61) (end 41.3 75.47259) (width 1) (layer "B.Cu") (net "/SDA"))
 (segment (start 46.721522 77.5) (end 30 77.5) (width 1) (layer "F.Cu") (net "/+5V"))
 (via (at 30 77.5) (size 0.6) (drill 0.3) (layers "F.Cu" "B.Cu") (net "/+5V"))
 (via (at 46.721522 77.5) (size 0.6) (drill 0.3) (layers "F.Cu" "B.Cu") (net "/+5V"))
 (segment (start 28.63904 77.5) (end 27.93632 76.79728) (width 1) (layer "B.Cu") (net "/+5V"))
 (segment (start 46.721522 77.5) (end 49.861522 80.64) (width 1) (layer "B.Cu") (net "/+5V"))
 (segment (start 55.36 29.64) (end 65.34 29.64) (width 1) (layer "B.Cu") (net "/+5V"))
 (segment (start 58.7 75.497056) (end 58.7 51.601472) (width 1) (layer "B.Cu") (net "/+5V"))
 (segment (start 58.7 51.601472) (end 53.8 46.701472) (width 1) (layer "B.Cu") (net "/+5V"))
 (segment (start 30 77.5) (end 28.63904 77.5) (width 1) (layer "B.Cu") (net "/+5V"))
 (segment (start 53.8 46.701472) (end 53.8 31.2) (width 1) (layer "B.Cu") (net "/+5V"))
 (segment (start 65.34 29.64) (end 73.48 21.5) (width 1) (layer "B.Cu") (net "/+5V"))
 (segment (start 53.557056 80.64) (end 58.7 75.497056) (width 1) (layer "B.Cu") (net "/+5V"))
 (segment (start 49.861522 80.64) (end 53.557056 80.64) (width 1) (layer "B.Cu") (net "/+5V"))
 (segment (start 53.8 31.2) (end 55.36 29.64) (width 1) (layer "B.Cu") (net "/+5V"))
 (segment (start 50.79728 79.33728) (end 50.8 79.34) (width 1) (layer "F.Cu") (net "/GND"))
 (segment (start 55 80) (end 55 76.8) (width 1) (layer "F.Cu") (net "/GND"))
 (segment (start 62.5 87.5) (end 55 80) (width 1) (layer "F.Cu") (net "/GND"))
 (segment (start 76.5 56) (end 57.5 75) (width 1) (layer "F.Cu") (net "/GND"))
 (segment (start 55 32.5) (end 55 27.5) (width 1) (layer "F.Cu") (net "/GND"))
 (segment (start 27.93632 79.33728) (end 50.79728 79.33728) (width 1) (layer "F.Cu") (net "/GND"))
 (via (at 57.5 75) (size 0.6) (drill 0.3) (layers "F.Cu" "B.Cu") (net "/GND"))
 (via (at 55 27.5) (size 0.6) (drill 0.3) (layers "F.Cu" "B.Cu") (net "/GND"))
 (via (at 55 76.8) (size 0.6) (drill 0.3) (layers "F.Cu" "B.Cu") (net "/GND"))
 (via (at 76.5 56) (size 0.6) (drill 0.3) (layers "F.Cu" "B.Cu") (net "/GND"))
 (via (at 62.5 87.5) (size 0.6) (drill 0.3) (layers "F.Cu" "B.Cu") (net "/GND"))
 (via (at 55 32.5) (size 0.6) (drill 0.3) (layers "F.Cu" "B.Cu") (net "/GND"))
 (segment (start 69.5 28.02) (end 76.02 21.5) (width 1) (layer "B.Cu") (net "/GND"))
 (segment (start 55 27.5) (end 53.5 26) (width 1) (layer "B.Cu") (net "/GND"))
 (segment (start 89.542081 85.04) (end 91.09 83.492081) (width 1) (layer "B.Cu") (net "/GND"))
 (segment (start 88.34 85.04) (end 89.542081 85.04) (width 1) (layer "B.Cu") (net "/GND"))
 (segment (start 74.64 88.7) (end 63.7 88.7) (width 1) (layer "B.Cu") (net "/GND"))
 (segment (start 58.84 33.73) (end 67.87 33.73) (width 1) (layer "B.Cu") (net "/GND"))
 (segment (start 78.3 85.04) (end 77.84 85.5) (width 1) (layer "B.Cu") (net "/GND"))
 (segment (start 69.5 32.1) (end 69.5 28.02) (width 1) (layer "B.Cu") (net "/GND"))
 (segment (start 88.34 85.04) (end 78.3 85.04) (width 1) (layer "B.Cu") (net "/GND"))
 (segment (start 53.5 26) (end 50.8 26) (width 1) (layer "B.Cu") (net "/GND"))
 (segment (start 67.87 33.73) (end 69.5 32.1) (width 1) (layer "B.Cu") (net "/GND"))
 (segment (start 76.5 56) (end 86.8 56) (width 1) (layer "B.Cu") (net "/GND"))
 (segment (start 78.06 23.54) (end 76.02 21.5) (width 1) (layer "B.Cu") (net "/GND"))
 (segment (start 55.7 76.8) (end 57.5 75) (width 1) (layer "B.Cu") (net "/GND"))
 (segment (start 50.8 79.34) (end 50.8 76.8) (width 1) (layer "B.Cu") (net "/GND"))
 (segment (start 86.8 56) (end 86.84 55.96) (width 1) (layer "B.Cu") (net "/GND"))
 (segment (start 55 32.5) (end 56.23 33.73) (width 1) (layer "B.Cu") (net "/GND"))
 (segment (start 63.7 88.7) (end 62.5 87.5) (width 1) (layer "B.Cu") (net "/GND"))
 (segment (start 50.8 76.8) (end 55 76.8) (width 1) (layer "B.Cu") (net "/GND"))
 (segment (start 91.09 83.492081) (end 91.09 36.57) (width 1) (layer "B.Cu") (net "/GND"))
 (segment (start 55 76.8) (end 55.7 76.8) (width 1) (layer "B.Cu") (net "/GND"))
 (segment (start 91.09 36.57) (end 78.06 23.54) (width 1) (layer "B.Cu") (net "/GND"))
 (segment (start 77.84 85.5) (end 74.64 88.7) (width 1) (layer "B.Cu") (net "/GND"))
 (segment (start 56.23 33.73) (end 58.84 33.73) (width 1) (layer "B.Cu") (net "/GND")))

